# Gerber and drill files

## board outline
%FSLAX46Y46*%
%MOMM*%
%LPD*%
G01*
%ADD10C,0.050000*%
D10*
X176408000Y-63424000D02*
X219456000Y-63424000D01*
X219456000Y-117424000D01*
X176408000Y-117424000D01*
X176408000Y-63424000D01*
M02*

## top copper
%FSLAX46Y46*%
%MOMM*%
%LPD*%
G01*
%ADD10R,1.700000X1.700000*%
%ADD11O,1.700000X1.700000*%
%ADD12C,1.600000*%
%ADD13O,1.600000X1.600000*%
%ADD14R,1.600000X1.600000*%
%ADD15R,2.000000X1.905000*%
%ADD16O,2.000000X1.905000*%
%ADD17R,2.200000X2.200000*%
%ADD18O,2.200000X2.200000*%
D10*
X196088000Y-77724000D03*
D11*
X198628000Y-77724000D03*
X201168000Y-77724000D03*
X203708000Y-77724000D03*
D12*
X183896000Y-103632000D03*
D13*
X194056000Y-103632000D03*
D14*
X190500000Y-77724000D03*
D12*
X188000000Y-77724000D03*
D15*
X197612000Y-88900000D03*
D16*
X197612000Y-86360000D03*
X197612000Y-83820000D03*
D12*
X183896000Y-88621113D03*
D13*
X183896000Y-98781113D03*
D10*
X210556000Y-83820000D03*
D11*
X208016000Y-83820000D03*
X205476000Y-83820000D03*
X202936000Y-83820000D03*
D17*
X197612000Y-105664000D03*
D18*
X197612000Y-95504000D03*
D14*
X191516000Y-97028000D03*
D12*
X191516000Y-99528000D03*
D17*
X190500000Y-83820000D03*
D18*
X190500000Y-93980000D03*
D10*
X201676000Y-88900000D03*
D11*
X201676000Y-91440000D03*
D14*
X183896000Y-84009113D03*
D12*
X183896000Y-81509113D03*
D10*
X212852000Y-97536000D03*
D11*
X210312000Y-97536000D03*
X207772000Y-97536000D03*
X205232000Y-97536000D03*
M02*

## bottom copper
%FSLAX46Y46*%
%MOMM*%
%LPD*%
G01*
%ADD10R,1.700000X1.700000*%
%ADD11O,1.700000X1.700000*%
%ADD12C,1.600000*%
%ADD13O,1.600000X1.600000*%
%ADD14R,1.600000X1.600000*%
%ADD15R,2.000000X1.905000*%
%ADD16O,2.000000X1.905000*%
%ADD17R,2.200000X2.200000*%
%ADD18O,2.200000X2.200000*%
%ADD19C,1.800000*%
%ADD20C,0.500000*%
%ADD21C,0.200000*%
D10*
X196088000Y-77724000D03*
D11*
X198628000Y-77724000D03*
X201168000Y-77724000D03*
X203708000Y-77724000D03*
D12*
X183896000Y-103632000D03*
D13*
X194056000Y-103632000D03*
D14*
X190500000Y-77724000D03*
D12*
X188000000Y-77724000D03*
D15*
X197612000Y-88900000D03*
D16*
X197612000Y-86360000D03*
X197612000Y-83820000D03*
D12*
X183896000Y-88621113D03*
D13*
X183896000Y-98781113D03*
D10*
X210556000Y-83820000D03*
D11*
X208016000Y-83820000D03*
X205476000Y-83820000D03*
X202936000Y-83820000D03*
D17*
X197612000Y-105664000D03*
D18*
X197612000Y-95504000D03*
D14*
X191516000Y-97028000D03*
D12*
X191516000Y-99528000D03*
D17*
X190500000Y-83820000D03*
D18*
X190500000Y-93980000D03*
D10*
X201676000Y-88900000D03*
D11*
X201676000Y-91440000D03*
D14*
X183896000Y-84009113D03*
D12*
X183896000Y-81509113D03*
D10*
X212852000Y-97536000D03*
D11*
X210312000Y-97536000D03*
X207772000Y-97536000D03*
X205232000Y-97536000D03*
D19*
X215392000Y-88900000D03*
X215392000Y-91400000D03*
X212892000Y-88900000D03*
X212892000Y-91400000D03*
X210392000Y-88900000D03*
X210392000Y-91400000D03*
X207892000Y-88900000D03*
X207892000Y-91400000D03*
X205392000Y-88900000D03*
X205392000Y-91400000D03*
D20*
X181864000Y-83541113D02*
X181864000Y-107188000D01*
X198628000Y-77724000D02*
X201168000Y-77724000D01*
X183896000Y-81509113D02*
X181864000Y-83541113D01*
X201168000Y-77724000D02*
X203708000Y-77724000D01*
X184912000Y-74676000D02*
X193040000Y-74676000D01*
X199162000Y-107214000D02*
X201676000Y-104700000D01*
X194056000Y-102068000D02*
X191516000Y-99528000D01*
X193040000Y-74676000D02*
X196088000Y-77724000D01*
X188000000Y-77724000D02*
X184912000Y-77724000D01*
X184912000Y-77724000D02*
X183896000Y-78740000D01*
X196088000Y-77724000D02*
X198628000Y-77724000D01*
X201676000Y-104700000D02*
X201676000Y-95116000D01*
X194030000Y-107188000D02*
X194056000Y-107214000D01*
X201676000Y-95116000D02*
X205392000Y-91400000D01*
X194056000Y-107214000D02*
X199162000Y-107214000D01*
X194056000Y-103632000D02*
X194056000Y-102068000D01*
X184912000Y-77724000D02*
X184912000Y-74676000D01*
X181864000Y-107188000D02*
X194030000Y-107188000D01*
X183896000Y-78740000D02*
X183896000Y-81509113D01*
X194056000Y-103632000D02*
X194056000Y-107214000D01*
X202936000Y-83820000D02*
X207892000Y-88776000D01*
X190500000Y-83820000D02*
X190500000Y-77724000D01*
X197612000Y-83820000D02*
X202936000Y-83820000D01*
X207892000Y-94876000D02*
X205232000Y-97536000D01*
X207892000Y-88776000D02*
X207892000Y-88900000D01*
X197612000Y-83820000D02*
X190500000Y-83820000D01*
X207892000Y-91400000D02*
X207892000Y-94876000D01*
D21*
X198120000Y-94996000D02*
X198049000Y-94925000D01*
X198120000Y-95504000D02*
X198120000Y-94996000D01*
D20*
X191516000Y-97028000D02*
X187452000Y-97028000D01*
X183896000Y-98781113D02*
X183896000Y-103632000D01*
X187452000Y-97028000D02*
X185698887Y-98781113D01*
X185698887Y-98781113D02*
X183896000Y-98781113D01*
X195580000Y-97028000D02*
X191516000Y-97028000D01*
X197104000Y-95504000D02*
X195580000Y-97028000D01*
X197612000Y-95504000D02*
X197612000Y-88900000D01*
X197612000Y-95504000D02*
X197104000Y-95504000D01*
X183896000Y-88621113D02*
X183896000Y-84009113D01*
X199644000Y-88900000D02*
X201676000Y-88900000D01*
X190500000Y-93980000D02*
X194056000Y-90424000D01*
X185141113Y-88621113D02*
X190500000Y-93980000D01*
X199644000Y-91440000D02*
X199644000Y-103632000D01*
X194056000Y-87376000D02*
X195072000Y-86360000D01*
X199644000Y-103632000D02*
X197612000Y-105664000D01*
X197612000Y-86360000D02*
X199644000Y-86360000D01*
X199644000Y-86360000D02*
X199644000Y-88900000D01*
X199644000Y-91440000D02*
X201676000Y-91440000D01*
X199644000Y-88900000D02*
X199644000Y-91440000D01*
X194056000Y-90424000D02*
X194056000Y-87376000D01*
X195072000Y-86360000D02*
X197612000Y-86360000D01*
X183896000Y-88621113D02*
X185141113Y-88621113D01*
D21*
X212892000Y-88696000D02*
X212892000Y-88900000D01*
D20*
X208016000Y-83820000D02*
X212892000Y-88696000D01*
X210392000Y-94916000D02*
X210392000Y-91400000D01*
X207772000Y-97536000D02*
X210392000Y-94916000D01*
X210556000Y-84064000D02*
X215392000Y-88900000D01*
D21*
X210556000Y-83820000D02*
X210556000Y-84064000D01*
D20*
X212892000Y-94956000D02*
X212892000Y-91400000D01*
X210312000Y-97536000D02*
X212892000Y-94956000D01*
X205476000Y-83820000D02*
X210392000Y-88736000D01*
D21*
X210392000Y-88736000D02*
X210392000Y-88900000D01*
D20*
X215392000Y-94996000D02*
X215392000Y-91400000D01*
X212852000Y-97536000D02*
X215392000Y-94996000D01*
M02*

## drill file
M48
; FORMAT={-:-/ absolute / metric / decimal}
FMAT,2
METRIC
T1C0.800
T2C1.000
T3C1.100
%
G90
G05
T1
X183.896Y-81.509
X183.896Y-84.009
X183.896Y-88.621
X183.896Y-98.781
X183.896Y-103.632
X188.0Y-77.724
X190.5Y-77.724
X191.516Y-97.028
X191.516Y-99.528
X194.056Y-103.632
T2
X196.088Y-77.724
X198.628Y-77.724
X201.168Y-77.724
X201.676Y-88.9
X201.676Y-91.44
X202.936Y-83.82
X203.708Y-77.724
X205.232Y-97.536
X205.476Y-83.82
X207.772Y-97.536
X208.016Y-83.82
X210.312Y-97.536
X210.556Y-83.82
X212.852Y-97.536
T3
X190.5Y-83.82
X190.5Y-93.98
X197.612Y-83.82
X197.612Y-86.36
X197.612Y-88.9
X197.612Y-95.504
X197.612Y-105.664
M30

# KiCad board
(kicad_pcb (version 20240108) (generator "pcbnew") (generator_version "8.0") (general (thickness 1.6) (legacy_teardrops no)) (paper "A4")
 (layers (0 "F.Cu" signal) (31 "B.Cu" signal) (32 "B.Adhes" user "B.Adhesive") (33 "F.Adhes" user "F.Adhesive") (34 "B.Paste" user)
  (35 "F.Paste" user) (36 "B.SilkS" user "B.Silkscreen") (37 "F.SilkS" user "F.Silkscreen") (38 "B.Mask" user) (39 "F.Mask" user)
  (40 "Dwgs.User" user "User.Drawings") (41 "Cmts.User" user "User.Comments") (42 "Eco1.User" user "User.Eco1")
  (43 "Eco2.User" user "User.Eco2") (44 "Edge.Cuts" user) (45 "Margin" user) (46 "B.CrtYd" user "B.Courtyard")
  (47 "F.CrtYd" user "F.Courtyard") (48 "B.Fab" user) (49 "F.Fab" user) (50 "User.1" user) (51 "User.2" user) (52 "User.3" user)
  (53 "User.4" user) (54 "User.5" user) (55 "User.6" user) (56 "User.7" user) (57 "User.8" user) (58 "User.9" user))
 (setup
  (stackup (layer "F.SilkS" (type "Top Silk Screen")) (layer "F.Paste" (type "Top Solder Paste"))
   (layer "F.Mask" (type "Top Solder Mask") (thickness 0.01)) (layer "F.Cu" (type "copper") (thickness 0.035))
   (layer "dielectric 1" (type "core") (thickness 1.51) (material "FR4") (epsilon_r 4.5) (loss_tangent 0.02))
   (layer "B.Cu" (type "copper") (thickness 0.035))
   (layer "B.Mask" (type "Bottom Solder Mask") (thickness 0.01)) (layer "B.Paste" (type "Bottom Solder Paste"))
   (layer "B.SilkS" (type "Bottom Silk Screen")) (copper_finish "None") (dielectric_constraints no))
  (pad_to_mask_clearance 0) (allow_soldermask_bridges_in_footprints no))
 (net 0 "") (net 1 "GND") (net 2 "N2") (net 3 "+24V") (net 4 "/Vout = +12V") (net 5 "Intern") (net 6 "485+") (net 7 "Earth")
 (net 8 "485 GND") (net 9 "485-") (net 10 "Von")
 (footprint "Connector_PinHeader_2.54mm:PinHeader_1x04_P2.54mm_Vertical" (layer "F.Cu") (at 196.088 77.724 90)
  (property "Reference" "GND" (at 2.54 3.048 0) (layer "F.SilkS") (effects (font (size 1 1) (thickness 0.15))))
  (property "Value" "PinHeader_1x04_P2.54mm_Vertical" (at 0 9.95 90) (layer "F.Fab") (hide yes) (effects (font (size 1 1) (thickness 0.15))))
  (pad "1" thru_hole rect (at 0 0 90) (size 1.7 1.7) (drill 1) (layers "*.Cu" "*.Mask") (remove_unused_layers no) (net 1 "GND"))
  (pad "2" thru_hole oval (at 0 2.54 90) (size 1.7 1.7) (drill 1) (layers "*.Cu" "*.Mask") (remove_unused_layers no) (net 1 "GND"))
  (pad "3" thru_hole oval (at 0 5.08 90) (size 1.7 1.7) (drill 1) (layers "*.Cu" "*.Mask") (remove_unused_layers no) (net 1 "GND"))
  (pad "4" thru_hole oval (at 0 7.62 90) (size 1.7 1.7) (drill 1) (layers "*.Cu" "*.Mask") (remove_unused_layers no) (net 1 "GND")))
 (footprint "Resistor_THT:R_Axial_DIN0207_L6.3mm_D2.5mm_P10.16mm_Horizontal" (layer "F.Cu") (at 183.896 103.632)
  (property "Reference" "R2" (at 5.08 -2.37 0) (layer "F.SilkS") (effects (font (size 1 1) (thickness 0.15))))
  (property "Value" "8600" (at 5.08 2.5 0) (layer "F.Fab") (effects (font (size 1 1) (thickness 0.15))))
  (pad "1" thru_hole circle (at 0 0) (size 1.6 1.6) (drill 0.8) (layers "*.Cu" "*.Mask") (remove_unused_layers no) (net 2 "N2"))
  (pad "2" thru_hole oval (at 10.16 0) (size 1.6 1.6) (drill 0.8) (layers "*.Cu" "*.Mask") (remove_unused_layers no) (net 1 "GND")))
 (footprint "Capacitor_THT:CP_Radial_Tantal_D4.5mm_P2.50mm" (layer "F.Cu") (at 190.5 77.724 180)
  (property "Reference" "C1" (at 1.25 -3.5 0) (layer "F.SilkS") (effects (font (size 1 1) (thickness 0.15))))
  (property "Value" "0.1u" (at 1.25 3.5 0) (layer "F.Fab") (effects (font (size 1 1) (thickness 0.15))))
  (pad "1" thru_hole rect (at 0 0 180) (size 1.6 1.6) (drill 0.8) (layers "*.Cu" "*.Mask") (remove_unused_layers no) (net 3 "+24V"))
  (pad "2" thru_hole circle (at 2.5 0 180) (size 1.6 1.6) (drill 0.8) (layers "*.Cu" "*.Mask") (remove_unused_layers no) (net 1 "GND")))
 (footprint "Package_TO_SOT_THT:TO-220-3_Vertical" (layer "F.Cu") (at 197.612 88.9 90)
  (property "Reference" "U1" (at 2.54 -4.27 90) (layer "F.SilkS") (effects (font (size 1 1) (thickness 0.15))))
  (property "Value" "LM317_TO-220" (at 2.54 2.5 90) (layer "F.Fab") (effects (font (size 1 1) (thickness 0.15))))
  (pad "1" thru_hole rect (at 0 0 90) (size 1.905 2) (drill 1.1) (layers "*.Cu" "*.Mask") (remove_unused_layers no) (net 2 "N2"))
  (pad "2" thru_hole oval (at 2.54 0 90) (size 1.905 2) (drill 1.1) (layers "*.Cu" "*.Mask") (remove_unused_layers no)
   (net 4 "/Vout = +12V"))
  (pad "3" thru_hole oval (at 5.08 0 90) (size 1.905 2) (drill 1.1) (layers "*.Cu" "*.Mask") (remove_unused_layers no) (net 3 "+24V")))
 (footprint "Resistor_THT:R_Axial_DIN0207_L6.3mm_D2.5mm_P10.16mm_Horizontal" (layer "F.Cu") (at 183.896 88.621113 -90)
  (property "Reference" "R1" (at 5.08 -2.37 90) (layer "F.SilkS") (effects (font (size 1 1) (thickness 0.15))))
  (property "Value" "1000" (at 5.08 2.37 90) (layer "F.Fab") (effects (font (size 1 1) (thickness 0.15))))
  (pad "1" thru_hole circle (at 0 0 270) (size 1.6 1.6) (drill 0.8) (layers "*.Cu" "*.Mask") (remove_unused_layers no)
   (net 4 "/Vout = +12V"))
  (pad "2" thru_hole oval (at 10.16 0 270) (size 1.6 1.6) (drill 0.8) (layers "*.Cu" "*.Mask") (remove_unused_layers no) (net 2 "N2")))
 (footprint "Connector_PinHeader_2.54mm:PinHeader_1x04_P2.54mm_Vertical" (layer "F.Cu") (at 210.556 83.82 -90)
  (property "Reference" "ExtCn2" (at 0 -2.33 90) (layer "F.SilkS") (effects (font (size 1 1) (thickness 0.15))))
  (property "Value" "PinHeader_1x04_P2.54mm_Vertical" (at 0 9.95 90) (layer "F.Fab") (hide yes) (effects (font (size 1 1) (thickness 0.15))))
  (pad "1" thru_hole rect (at 0 0 270) (size 1.7 1.7) (drill 1) (layers "*.Cu" "*.Mask" "B.Paste") (remove_unused_layers no)
   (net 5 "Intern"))
  (pad "2" thru_hole oval (at 0 2.54 270) (size 1.7 1.7) (drill 1) (layers "*.Cu" "*.Mask") (remove_unused_layers no) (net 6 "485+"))
  (pad "3" thru_hole oval (at 0 5.08 270) (size 1.7 1.7) (drill 1) (layers "*.Cu" "*.Mask" "Eco1.User") (remove_unused_layers no)
   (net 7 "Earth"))
  (pad "4" thru_hole oval (at 0 7.62 270) (size 1.7 1.7) (drill 1) (layers "*.Cu" "*.Mask") (remove_unused_layers no) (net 3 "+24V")))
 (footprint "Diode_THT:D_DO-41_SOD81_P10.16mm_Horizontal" (layer "F.Cu") (at 197.612 105.664 90)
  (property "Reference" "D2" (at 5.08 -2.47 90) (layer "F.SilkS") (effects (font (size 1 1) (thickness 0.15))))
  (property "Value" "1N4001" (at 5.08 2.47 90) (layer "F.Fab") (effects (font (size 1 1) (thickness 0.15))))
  (pad "1" thru_hole rect (at 0 0 90) (size 2.2 2.2) (drill 1.1) (layers "*.Cu" "*.Mask") (remove_unused_layers no) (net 4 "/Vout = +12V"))
  (pad "2" thru_hole oval (at 10.16 0 90) (size 2.2 2.2) (drill 1.1) (layers "*.Cu" "*.Mask") (remove_unused_layers no) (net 2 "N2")))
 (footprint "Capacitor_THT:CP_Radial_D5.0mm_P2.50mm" (layer "F.Cu") (at 191.516 97.028 -90)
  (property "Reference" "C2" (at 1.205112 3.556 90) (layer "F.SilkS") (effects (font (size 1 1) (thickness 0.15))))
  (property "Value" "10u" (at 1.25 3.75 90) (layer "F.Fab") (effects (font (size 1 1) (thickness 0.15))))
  (pad "1" thru_hole rect (at 0 0 270) (size 1.6 1.6) (drill 0.8) (layers "*.Cu" "*.Mask") (remove_unused_layers no) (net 2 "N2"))
  (pad "2" thru_hole circle (at 2.5 0 270) (size 1.6 1.6) (drill 0.8) (layers "*.Cu" "*.Mask") (remove_unused_layers no) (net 1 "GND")))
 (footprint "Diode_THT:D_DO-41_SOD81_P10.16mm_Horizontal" (layer "F.Cu") (at 190.5 83.82 -90)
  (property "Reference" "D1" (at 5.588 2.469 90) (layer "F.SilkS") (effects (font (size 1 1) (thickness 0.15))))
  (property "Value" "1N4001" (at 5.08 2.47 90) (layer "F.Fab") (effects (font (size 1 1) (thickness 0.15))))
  (pad "1" thru_hole rect (at 0 0 270) (size 2.2 2.2) (drill 1.1) (layers "*.Cu" "*.Mask") (remove_unused_layers no) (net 3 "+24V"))
  (pad "2" thru_hole oval (at 10.16 0 270) (size 2.2 2.2) (drill 1.1) (layers "*.Cu" "*.Mask") (remove_unused_layers no)
   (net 4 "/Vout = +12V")))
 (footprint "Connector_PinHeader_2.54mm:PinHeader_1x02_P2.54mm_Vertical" (layer "F.Cu") (at 201.676 88.9)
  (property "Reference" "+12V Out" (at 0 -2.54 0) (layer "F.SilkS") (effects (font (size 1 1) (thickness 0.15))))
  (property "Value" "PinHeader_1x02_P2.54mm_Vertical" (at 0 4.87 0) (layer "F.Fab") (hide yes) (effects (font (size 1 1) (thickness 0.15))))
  (pad "1" thru_hole rect (at 0 0) (size 1.7 1.7) (drill 1) (layers "*.Cu" "*.Mask") (remove_unused_layers no) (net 4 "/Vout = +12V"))
  (pad "2" thru_hole oval (at 0 2.54) (size 1.7 1.7) (drill 1) (layers "*.Cu" "*.Mask") (remove_unused_layers no) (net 4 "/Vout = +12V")))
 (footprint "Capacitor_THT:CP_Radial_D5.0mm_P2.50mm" (layer "F.Cu") (at 183.896 84.009113 90)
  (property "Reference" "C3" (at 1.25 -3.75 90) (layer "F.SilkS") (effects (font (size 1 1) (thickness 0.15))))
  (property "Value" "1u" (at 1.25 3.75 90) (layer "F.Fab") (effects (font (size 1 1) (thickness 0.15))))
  (pad "1" thru_hole rect (at 0 0 90) (size 1.6 1.6) (drill 0.8) (layers "*.Cu" "*.Mask") (remove_unused_layers no) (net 4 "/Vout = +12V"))
  (pad "2" thru_hole circle (at 2.5 0 90) (size 1.6 1.6) (drill 0.8) (layers "*.Cu" "*.Mask") (remove_unused_layers no) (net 1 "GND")))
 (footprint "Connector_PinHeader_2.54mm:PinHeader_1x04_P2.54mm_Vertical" (layer "F.Cu") (at 212.852 97.536 -90)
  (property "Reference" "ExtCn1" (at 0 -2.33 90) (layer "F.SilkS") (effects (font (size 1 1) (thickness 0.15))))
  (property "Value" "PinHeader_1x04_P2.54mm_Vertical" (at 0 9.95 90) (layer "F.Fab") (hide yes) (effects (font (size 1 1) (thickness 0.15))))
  (pad "1" thru_hole rect (at 0 0 270) (size 1.7 1.7) (drill 1) (layers "*.Cu" "*.Mask") (remove_unused_layers no) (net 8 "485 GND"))
  (pad "2" thru_hole oval (at 0 2.54 270) (size 1.7 1.7) (drill 1) (layers "*.Cu" "*.Mask") (remove_unused_layers no) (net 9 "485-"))
  (pad "3" thru_hole oval (at 0 5.08 270) (size 1.7 1.7) (drill 1) (layers "*.Cu" "*.Mask") (remove_unused_layers no) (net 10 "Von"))
  (pad "4" thru_hole oval (at 0 7.62 270) (size 1.7 1.7) (drill 1) (layers "*.Cu" "*.Mask") (remove_unused_layers no) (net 3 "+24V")))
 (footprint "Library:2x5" (layer "B.Cu") (at 215.392 88.9 180)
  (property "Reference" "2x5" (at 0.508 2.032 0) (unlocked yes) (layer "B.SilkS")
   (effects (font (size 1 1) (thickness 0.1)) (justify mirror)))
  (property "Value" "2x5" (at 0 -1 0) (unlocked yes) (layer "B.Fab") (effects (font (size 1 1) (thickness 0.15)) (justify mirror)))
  (pad "1" smd circle (at 0 0 180) (size 1.8 1.8) (layers "B.Cu" "B.Mask") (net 5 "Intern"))
  (pad "2" smd circle (at 0 -2.5 180) (size 1.8 1.8) (layers "B.Cu" "F.SilkS" "B.Mask") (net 8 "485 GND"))
  (pad "3" smd circle (at 2.5 0 180) (size 1.8 1.8) (layers "B.Cu" "B.Mask") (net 6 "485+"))
  (pad "4" smd circle (at 2.5 -2.5 180) (size 1.8 1.8) (layers "B.Cu" "B.Mask") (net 9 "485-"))
  (pad "5" smd circle (at 5 0 180) (size 1.8 1.8) (layers "B.Cu" "B.Mask") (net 7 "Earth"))
  (pad "6" smd circle (at 5 -2.5 180) (size 1.8 1.8) (layers "B.Cu" "B.Mask") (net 10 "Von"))
  (pad "7" smd circle (at 7.5 0 180) (size 1.8 1.8) (layers "B.Cu" "B.Mask") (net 3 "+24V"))
  (pad "8" smd circle (at 7.5 -2.5 180) (size 1.8 1.8) (layers "B.Cu" "B.Mask") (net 3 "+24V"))
  (pad "9" smd circle (at 10 0 180) (size 1.8 1.8) (layers "B.Cu" "B.Mask") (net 1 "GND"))
  (pad "10" smd circle (at 10 -2.5 180) (size 1.8 1.8) (layers "B.Cu" "B.Mask") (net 1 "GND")))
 (gr_rect (start 176.408 63.424) (end 219.456 117.424) (stroke (width 0.05) (type default)) (fill none) (layer "Edge.Cuts"))
 (segment (start 181.864 83.541113) (end 181.864 107.188) (width 0.5) (layer "B.Cu") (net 1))
 (segment (start 198.628 77.724) (end 201.168 77.724) (width 0.5) (layer "B.Cu") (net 1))
 (segment (start 183.896 81.509113) (end 181.864 83.541113) (width 0.5) (layer "B.Cu") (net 1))
 (segment (start 201.168 77.724) (end 203.708 77.724) (width 0.5) (layer "B.Cu") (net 1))
 (segment (start 184.912 74.676) (end 193.04 74.676) (width 0.5) (layer "B.Cu") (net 1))
 (segment (start 199.162 107.214) (end 201.676 104.7) (width 0.5) (layer "B.Cu") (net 1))
 (segment (start 194.056 102.068) (end 191.516 99.528) (width 0.5) (layer "B.Cu") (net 1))
 (segment (start 193.04 74.676) (end 196.088 77.724) (width 0.5) (layer "B.Cu") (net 1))
 (segment (start 188 77.724) (end 184.912 77.724) (width 0.5) (layer "B.Cu") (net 1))
 (segment (start 184.912 77.724) (end 183.896 78.74) (width 0.5) (layer "B.Cu") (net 1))
 (segment (start 196.088 77.724) (end 198.628 77.724) (width 0.5) (layer "B.Cu") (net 1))
 (segment (start 201.676 104.7) (end 201.676 95.116) (width 0.5) (layer "B.Cu") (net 1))
 (segment (start 194.03 107.188) (end 194.056 107.214) (width 0.5) (layer "B.Cu") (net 1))
 (segment (start 201.676 95.116) (end 205.392 91.4) (width 0.5) (layer "B.Cu") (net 1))
 (segment (start 194.056 107.214) (end 199.162 107.214) (width 0.5) (layer "B.Cu") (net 1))
 (segment (start 194.056 103.632) (end 194.056 102.068) (width 0.5) (layer "B.Cu") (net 1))
 (segment (start 184.912 77.724) (end 184.912 74.676) (width 0.5) (layer "B.Cu") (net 1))
 (segment (start 181.864 107.188) (end 194.03 107.188) (width 0.5) (layer "B.Cu") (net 1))
 (segment (start 183.896 78.74) (end 183.896 81.509113) (width 0.5) (layer "B.Cu") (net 1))
 (segment (start 194.056 103.632) (end 194.056 107.214) (width 0.5) (layer "B.Cu") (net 1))
 (segment (start 202.936 83.82) (end 207.892 88.776) (width 0.5) (layer "B.Cu") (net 3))
 (segment (start 190.5 83.82) (end 190.5 77.724) (width 0.5) (layer "B.Cu") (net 3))
 (segment (start 197.612 83.82) (end 202.936 83.82) (width 0.5) (layer "B.Cu") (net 3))
 (segment (start 207.892 94.876) (end 205.232 97.536) (width 0.5) (layer "B.Cu") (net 3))
 (segment (start 207.892 88.776) (end 207.892 88.9) (width 0.5) (layer "B.Cu") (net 3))
 (segment (start 197.612 83.82) (end 190.5 83.82) (width 0.5) (layer "B.Cu") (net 3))
 (segment (start 207.892 91.4) (end 207.892 94.876) (width 0.5) (layer "B.Cu") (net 3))
 (segment (start 198.12 94.996) (end 198.049 94.925) (width 0.2) (layer "B.Cu") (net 2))
 (segment (start 198.12 95.504) (end 198.12 94.996) (width 0.2) (layer "B.Cu") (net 2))
 (segment (start 191.516 97.028) (end 187.452 97.028) (width 0.5) (layer "B.Cu") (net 2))
 (segment (start 183.896 98.781113) (end 183.896 103.632) (width 0.5) (layer "B.Cu") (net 2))
 (segment (start 187.452 97.028) (end 185.698887 98.781113) (width 0.5) (layer "B.Cu") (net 2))
 (segment (start 185.698887 98.781113) (end 183.896 98.781113) (width 0.5) (layer "B.Cu") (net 2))
 (segment (start 195.58 97.028) (end 191.516 97.028) (width 0.5) (layer "B.Cu") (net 2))
 (segment (start 197.104 95.504) (end 195.58 97.028) (width 0.5) (layer "B.Cu") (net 2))
 (segment (start 197.612 95.504) (end 197.612 88.9) (width 0.5) (layer "B.Cu") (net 2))
 (segment (start 197.612 95.504) (end 197.104 95.504) (width 0.5) (layer "B.Cu") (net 2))
 (segment (start 183.896 88.621113) (end 183.896 84.009113) (width 0.5) (layer "B.Cu") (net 4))
 (segment (start 199.644 88.9) (end 201.676 88.9) (width 0.5) (layer "B.Cu") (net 4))
 (segment (start 190.5 93.98) (end 194.056 90.424) (width 0.5) (layer "B.Cu") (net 4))
 (segment (start 185.141113 88.621113) (end 190.5 93.98) (width 0.5) (layer "B.Cu") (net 4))
 (segment (start 199.644 91.44) (end 199.644 103.632) (width 0.5) (layer "B.Cu") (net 4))
 (segment (start 194.056 87.376) (end 195.072 86.36) (width 0.5) (layer "B.Cu") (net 4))
 (segment (start 199.644 103.632) (end 197.612 105.664) (width 0.5) (layer "B.Cu") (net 4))
 (segment (start 197.612 86.36) (end 199.644 86.36) (width 0.5) (layer "B.Cu") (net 4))
 (segment (start 199.644 86.36) (end 199.644 88.9) (width 0.5) (layer "B.Cu") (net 4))
 (segment (start 199.644 91.44) (end 201.676 91.44) (width 0.5) (layer "B.Cu") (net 4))
 (segment (start 199.644 88.9) (end 199.644 91.44) (width 0.5) (layer "B.Cu") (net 4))
 (segment (start 194.056 90.424) (end 194.056 87.376) (width 0.5) (layer "B.Cu") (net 4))
 (segment (start 195.072 86.36) (end 197.612 86.36) (width 0.5) (layer "B.Cu") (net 4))
 (segment (start 183.896 88.621113) (end 185.141113 88.621113) (width 0.5) (layer "B.Cu") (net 4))
 (segment (start 212.892 88.696) (end 212.892 88.9) (width 0.2) (layer "B.Cu") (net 6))
 (segment (start 208.016 83.82) (end 212.892 88.696) (width 0.5) (layer "B.Cu") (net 6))
 (segment (start 210.392 94.916) (end 210.392 91.4) (width 0.5) (layer "B.Cu") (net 10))
 (segment (start 207.772 97.536) (end 210.392 94.916) (width 0.5) (layer "B.Cu") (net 10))
 (segment (start 210.556 84.064) (end 215.392 88.9) (width 0.5) (layer "B.Cu") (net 5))
 (segment (start 210.556 83.82) (end 210.556 84.064) (width 0.2) (layer "B.Cu") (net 5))
 (segment (start 212.892 94.956) (end 212.892 91.4) (width 0.5) (layer "B.Cu") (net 9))
 (segment (start 210.312 97.536) (end 212.892 94.956) (width 0.5) (layer "B.Cu") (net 9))
 (segment (start 205.476 83.82) (end 210.392 88.736) (width 0.5) (layer "B.Cu") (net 7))
 (segment (start 210.392 88.736) (end 210.392 88.9) (width 0.2) (layer "B.Cu") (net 7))
 (segment (start 215.392 94.996) (end 215.392 91.4) (width 0.5) (layer "B.Cu") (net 8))
 (segment (start 212.852 97.536) (end 215.392 94.996) (width 0.5) (layer "B.Cu") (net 8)))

